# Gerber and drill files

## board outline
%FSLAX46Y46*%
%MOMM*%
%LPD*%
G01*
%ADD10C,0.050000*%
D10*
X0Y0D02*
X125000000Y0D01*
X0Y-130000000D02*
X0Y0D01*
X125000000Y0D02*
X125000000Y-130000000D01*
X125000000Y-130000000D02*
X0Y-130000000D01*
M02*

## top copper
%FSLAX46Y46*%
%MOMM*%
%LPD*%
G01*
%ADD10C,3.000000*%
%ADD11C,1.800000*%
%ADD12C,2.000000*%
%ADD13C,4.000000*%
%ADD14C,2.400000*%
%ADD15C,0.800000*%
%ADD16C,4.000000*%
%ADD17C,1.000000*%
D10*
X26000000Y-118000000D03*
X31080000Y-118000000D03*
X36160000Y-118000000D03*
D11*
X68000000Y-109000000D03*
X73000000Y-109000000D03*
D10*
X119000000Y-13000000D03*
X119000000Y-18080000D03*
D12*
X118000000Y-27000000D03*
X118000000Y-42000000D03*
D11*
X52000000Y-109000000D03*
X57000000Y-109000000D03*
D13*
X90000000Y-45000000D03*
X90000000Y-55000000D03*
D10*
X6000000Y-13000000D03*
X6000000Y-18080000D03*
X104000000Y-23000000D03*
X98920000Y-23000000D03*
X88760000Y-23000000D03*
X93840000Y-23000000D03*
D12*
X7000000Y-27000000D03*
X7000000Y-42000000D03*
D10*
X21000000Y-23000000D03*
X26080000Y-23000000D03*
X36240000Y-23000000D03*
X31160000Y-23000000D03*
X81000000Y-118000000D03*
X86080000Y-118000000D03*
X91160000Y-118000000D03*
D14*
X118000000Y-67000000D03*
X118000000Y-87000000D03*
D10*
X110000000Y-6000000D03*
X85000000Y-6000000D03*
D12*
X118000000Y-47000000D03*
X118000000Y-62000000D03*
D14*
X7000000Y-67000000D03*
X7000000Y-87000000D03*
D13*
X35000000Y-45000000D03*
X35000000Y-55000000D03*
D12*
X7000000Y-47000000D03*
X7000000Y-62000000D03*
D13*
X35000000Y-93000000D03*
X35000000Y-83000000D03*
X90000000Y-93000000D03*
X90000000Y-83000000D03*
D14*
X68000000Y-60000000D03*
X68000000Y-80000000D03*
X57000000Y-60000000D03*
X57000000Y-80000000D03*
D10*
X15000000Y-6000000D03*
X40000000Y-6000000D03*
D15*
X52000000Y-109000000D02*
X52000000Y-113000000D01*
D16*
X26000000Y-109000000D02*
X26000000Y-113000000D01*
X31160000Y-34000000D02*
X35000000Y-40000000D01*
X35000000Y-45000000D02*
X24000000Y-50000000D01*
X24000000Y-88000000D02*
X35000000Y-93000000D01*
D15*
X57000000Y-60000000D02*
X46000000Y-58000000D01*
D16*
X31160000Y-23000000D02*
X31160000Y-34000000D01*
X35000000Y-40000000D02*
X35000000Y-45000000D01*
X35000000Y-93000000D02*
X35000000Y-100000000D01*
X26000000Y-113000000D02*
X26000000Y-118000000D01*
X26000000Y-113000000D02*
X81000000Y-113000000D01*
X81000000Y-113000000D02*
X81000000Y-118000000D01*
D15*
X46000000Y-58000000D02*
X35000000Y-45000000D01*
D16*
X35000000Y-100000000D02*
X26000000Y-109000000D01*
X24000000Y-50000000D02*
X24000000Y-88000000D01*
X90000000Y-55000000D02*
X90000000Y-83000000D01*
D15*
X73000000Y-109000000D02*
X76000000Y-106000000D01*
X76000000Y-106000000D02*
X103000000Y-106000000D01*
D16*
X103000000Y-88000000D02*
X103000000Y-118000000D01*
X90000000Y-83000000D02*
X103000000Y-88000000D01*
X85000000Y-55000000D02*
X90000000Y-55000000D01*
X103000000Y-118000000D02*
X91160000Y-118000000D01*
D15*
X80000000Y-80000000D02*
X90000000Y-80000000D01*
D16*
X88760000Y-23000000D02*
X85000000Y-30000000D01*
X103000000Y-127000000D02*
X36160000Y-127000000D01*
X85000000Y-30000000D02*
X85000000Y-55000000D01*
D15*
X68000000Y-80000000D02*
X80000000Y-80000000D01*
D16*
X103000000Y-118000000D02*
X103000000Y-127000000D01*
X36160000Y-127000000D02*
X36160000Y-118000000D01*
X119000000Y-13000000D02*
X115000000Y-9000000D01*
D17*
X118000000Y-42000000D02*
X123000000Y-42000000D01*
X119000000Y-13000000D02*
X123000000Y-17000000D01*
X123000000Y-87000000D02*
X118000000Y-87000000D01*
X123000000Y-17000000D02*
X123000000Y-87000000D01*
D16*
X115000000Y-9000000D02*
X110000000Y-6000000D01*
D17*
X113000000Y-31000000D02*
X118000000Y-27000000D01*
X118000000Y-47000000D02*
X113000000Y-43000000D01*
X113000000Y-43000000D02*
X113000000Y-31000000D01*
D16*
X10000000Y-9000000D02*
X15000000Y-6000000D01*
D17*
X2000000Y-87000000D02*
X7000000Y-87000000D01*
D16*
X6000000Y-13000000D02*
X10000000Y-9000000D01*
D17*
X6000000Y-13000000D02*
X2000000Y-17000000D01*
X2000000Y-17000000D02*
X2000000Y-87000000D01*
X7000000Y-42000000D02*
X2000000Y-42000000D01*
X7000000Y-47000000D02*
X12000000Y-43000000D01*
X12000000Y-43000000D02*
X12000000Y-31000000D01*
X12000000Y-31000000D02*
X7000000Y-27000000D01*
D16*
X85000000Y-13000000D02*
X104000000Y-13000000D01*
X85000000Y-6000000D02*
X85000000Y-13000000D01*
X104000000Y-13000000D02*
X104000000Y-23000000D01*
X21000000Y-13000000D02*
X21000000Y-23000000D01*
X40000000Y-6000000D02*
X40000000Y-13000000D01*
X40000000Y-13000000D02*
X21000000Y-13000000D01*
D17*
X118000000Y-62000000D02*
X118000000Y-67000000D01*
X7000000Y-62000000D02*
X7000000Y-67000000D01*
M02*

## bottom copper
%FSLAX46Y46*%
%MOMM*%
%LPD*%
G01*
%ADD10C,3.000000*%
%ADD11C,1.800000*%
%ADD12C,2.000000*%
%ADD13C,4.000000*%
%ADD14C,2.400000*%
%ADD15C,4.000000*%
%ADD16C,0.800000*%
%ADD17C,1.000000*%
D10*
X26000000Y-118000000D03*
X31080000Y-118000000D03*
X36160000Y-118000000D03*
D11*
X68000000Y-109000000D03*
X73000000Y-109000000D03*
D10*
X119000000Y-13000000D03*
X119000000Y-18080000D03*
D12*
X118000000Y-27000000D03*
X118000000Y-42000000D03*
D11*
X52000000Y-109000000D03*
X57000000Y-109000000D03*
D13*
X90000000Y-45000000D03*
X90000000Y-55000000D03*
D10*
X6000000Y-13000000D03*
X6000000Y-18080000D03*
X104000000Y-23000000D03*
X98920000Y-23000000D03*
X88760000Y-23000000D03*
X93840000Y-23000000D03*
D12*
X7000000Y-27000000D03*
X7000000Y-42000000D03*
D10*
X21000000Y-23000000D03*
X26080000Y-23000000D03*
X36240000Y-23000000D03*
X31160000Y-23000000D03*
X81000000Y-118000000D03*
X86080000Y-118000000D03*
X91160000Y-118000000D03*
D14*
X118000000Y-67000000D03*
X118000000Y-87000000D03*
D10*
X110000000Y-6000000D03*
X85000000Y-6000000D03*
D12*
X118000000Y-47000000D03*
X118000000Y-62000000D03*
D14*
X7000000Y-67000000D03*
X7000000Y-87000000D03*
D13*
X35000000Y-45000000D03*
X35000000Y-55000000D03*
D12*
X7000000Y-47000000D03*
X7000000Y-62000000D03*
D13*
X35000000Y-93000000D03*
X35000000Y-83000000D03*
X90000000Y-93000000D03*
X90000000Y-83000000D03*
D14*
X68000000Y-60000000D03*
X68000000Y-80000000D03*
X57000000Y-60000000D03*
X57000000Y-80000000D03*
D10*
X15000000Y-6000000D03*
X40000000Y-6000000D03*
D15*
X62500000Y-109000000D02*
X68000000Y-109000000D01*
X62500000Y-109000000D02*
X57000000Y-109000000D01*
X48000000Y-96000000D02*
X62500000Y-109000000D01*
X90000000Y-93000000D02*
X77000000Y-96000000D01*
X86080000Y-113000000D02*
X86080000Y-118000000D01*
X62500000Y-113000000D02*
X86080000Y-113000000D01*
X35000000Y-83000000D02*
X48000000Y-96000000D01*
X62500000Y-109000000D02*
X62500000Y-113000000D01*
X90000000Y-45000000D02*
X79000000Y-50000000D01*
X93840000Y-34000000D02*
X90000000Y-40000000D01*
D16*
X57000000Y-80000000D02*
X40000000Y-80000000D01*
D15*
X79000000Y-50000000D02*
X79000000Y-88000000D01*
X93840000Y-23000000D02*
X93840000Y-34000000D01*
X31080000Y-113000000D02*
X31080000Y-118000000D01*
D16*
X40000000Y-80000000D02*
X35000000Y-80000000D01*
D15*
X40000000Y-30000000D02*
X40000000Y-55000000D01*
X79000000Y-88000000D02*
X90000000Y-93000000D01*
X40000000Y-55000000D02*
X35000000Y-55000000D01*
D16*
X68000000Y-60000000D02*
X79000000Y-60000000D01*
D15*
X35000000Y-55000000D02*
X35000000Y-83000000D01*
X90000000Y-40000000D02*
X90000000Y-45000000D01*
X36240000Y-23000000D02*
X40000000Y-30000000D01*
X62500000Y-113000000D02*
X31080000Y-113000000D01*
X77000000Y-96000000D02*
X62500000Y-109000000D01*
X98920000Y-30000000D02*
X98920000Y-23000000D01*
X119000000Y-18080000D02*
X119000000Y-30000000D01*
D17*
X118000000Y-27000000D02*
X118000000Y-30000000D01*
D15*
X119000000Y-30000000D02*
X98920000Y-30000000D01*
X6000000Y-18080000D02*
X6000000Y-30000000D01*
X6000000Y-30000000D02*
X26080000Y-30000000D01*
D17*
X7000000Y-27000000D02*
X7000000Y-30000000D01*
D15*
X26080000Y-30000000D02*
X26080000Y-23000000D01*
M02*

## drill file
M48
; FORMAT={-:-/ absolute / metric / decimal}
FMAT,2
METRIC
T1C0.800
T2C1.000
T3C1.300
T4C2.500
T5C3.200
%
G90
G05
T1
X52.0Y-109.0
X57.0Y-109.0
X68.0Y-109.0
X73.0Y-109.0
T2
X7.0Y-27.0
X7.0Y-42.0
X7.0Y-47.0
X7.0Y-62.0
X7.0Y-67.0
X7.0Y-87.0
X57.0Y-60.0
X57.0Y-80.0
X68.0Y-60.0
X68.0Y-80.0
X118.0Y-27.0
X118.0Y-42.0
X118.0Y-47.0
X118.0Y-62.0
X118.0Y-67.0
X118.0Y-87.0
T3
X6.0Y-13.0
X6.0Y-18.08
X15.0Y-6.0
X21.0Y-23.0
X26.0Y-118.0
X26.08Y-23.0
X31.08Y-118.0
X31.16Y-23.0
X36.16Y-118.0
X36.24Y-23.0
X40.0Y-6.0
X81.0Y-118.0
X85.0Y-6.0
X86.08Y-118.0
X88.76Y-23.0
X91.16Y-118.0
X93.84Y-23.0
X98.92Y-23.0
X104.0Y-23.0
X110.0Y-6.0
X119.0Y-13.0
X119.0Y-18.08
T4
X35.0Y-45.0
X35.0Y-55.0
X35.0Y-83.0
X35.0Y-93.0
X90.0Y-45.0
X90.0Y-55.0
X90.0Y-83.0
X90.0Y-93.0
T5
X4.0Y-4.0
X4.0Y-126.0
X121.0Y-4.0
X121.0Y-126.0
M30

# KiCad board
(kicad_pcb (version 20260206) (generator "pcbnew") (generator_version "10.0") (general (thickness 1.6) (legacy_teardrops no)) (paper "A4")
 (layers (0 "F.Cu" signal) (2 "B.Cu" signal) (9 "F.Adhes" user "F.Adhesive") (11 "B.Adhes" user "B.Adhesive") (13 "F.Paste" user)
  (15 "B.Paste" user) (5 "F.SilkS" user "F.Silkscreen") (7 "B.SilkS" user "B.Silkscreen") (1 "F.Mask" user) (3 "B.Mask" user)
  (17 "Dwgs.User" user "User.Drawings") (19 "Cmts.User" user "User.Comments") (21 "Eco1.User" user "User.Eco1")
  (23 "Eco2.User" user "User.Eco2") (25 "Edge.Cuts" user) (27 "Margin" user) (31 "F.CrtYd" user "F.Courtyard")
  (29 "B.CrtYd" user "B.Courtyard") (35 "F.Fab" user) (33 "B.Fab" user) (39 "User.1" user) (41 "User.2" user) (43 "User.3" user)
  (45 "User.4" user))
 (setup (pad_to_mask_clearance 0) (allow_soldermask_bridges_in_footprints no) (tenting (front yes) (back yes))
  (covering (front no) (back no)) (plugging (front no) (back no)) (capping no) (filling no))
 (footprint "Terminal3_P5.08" (layer "F.Cu") (at 26 118)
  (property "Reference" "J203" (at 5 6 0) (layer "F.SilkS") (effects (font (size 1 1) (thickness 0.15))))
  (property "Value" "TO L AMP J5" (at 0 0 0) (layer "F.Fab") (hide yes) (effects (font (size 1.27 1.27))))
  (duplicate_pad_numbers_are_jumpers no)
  (pad "1" thru_hole circle (at 0 0) (size 3 3) (drill 1.3) (layers "*.Cu" "*.Mask") (remove_unused_layers no) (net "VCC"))
  (pad "2" thru_hole circle (at 5.08 0) (size 3 3) (drill 1.3) (layers "*.Cu" "*.Mask") (remove_unused_layers no) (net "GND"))
  (pad "3" thru_hole circle (at 10.16 0) (size 3 3) (drill 1.3) (layers "*.Cu" "*.Mask") (remove_unused_layers no) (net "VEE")))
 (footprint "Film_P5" (layer "F.Cu") (at 68 109)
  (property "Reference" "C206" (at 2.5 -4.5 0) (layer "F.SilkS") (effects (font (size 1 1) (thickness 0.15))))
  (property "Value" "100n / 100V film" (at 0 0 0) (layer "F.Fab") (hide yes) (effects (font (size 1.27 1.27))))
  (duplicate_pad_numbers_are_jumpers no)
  (pad "1" thru_hole circle (at 0 0) (size 1.8 1.8) (drill 0.8) (layers "*.Cu" "*.Mask") (remove_unused_layers no) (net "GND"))
  (pad "2" thru_hole circle (at 5 0) (size 1.8 1.8) (drill 0.8) (layers "*.Cu" "*.Mask") (remove_unused_layers no) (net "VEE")))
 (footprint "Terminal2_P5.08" (layer "F.Cu") (at 119 13 -90)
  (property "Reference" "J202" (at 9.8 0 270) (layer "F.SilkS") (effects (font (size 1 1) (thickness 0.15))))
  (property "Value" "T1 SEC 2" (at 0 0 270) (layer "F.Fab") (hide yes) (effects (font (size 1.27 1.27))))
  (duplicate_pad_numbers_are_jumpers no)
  (pad "1" thru_hole circle (at 0 0 270) (size 3 3) (drill 1.3) (layers "*.Cu" "*.Mask") (remove_unused_layers no) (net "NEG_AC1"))
  (pad "2" thru_hole circle (at 5.08 0 270) (size 3 3) (drill 1.3) (layers "*.Cu" "*.Mask") (remove_unused_layers no) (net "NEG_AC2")))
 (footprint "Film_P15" (layer "F.Cu") (at 118 27 -90)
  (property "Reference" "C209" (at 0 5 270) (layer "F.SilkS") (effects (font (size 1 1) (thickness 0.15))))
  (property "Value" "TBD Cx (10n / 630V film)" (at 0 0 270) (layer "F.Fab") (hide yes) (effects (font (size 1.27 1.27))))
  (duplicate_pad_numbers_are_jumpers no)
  (pad "1" thru_hole circle (at 0 0 270) (size 2 2) (drill 1) (layers "*.Cu" "*.Mask") (remove_unused_layers no) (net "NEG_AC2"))
  (pad "2" thru_hole circle (at 15 0 270) (size 2 2) (drill 1) (layers "*.Cu" "*.Mask") (remove_unused_layers no) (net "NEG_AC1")))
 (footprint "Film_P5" (layer "F.Cu") (at 52 109)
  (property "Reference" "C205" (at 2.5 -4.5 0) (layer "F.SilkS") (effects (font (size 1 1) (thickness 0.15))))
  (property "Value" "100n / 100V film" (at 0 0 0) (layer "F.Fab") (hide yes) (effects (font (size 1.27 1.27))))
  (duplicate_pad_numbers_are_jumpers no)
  (pad "1" thru_hole circle (at 0 0) (size 1.8 1.8) (drill 0.8) (layers "*.Cu" "*.Mask") (remove_unused_layers no) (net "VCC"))
  (pad "2" thru_hole circle (at 5 0) (size 1.8 1.8) (drill 0.8) (layers "*.Cu" "*.Mask") (remove_unused_layers no) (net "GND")))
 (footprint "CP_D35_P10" (layer "F.Cu") (at 90 45 -90)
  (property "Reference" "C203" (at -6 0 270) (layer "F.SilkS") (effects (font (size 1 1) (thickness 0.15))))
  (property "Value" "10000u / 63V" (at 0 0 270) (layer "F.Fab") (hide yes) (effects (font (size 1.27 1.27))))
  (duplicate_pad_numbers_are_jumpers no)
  (pad "1" thru_hole circle (at 0 0 270) (size 4 4) (drill 2.5) (layers "*.Cu" "*.Mask") (remove_unused_layers no) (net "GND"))
  (pad "2" thru_hole circle (at 10 0 270) (size 4 4) (drill 2.5) (layers "*.Cu" "*.Mask") (remove_unused_layers no) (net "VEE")))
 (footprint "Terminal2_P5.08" (layer "F.Cu") (at 6 13 -90)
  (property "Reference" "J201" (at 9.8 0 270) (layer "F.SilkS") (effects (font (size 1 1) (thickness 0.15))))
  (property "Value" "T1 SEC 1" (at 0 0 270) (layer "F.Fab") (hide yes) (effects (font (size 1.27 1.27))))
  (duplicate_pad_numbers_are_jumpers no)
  (pad "1" thru_hole circle (at 0 0 270) (size 3 3) (drill 1.3) (layers "*.Cu" "*.Mask") (remove_unused_layers no) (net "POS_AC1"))
  (pad "2" thru_hole circle (at 5.08 0 270) (size 3 3) (drill 1.3) (layers "*.Cu" "*.Mask") (remove_unused_layers no) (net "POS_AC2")))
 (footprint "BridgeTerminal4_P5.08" (layer "F.Cu") (at 104 23 180)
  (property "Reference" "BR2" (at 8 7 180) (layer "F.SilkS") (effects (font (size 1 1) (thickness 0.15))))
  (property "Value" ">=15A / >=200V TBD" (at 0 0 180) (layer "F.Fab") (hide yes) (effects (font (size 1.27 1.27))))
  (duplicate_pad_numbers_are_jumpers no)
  (pad "AC1" thru_hole circle (at 0 0 180) (size 3 3) (drill 1.3) (layers "*.Cu" "*.Mask") (remove_unused_layers no) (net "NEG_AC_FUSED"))
  (pad "AC2" thru_hole circle (at 5.08 0 180) (size 3 3) (drill 1.3) (layers "*.Cu" "*.Mask") (remove_unused_layers no) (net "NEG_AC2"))
  (pad "N" thru_hole circle (at 15.24 0 180) (size 3 3) (drill 1.3) (layers "*.Cu" "*.Mask") (remove_unused_layers no) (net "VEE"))
  (pad "P" thru_hole circle (at 10.16 0 180) (size 3 3) (drill 1.3) (layers "*.Cu" "*.Mask") (remove_unused_layers no) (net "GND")))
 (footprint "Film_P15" (layer "F.Cu") (at 7 27 -90)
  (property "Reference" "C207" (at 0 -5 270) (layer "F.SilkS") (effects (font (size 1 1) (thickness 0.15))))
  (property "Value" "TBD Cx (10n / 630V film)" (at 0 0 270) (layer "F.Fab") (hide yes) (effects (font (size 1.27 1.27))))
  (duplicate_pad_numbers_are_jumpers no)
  (pad "1" thru_hole circle (at 0 0 270) (size 2 2) (drill 1) (layers "*.Cu" "*.Mask") (remove_unused_layers no) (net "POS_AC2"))
  (pad "2" thru_hole circle (at 15 0 270) (size 2 2) (drill 1) (layers "*.Cu" "*.Mask") (remove_unused_layers no) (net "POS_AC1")))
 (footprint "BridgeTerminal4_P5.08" (layer "F.Cu") (at 21 23)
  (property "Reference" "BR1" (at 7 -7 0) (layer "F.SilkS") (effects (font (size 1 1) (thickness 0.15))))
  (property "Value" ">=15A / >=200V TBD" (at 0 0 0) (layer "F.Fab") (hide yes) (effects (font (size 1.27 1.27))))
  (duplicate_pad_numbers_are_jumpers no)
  (pad "AC1" thru_hole circle (at 0 0) (size 3 3) (drill 1.3) (layers "*.Cu" "*.Mask") (remove_unused_layers no) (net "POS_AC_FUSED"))
  (pad "AC2" thru_hole circle (at 5.08 0) (size 3 3) (drill 1.3) (layers "*.Cu" "*.Mask") (remove_unused_layers no) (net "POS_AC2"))
  (pad "N" thru_hole circle (at 15.24 0) (size 3 3) (drill 1.3) (layers "*.Cu" "*.Mask") (remove_unused_layers no) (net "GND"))
  (pad "P" thru_hole circle (at 10.16 0) (size 3 3) (drill 1.3) (layers "*.Cu" "*.Mask") (remove_unused_layers no) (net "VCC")))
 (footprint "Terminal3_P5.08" (layer "F.Cu") (at 81 118)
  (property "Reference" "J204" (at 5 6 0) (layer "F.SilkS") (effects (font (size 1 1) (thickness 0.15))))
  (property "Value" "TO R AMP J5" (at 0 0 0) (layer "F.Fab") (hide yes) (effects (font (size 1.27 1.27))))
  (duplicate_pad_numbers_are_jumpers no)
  (pad "1" thru_hole circle (at 0 0) (size 3 3) (drill 1.3) (layers "*.Cu" "*.Mask") (remove_unused_layers no) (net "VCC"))
  (pad "2" thru_hole circle (at 5.08 0) (size 3 3) (drill 1.3) (layers "*.Cu" "*.Mask") (remove_unused_layers no) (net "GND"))
  (pad "3" thru_hole circle (at 10.16 0) (size 3 3) (drill 1.3) (layers "*.Cu" "*.Mask") (remove_unused_layers no) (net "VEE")))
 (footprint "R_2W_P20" (layer "F.Cu") (at 118 67 -90)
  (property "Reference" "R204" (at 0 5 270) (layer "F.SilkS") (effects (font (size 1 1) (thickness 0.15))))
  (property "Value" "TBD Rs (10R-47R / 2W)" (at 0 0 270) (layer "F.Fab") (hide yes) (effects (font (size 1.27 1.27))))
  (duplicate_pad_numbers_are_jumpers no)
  (pad "1" thru_hole circle (at 0 0 270) (size 2.4 2.4) (drill 1) (layers "*.Cu" "*.Mask") (remove_unused_layers no) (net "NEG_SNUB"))
  (pad "2" thru_hole circle (at 20 0 270) (size 2.4 2.4) (drill 1) (layers "*.Cu" "*.Mask") (remove_unused_layers no) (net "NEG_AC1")))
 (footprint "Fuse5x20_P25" (layer "F.Cu") (at 110 6 180)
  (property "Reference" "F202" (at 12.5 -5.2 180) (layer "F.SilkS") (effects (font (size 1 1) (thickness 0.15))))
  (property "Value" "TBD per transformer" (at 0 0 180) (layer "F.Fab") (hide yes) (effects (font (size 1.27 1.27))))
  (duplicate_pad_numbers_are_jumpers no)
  (pad "1" thru_hole circle (at 0 0 180) (size 3 3) (drill 1.3) (layers "*.Cu" "*.Mask") (remove_unused_layers no) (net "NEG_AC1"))
  (pad "2" thru_hole circle (at 25 0 180) (size 3 3) (drill 1.3) (layers "*.Cu" "*.Mask") (remove_unused_layers no) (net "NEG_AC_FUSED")))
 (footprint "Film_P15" (layer "F.Cu") (at 118 47 -90)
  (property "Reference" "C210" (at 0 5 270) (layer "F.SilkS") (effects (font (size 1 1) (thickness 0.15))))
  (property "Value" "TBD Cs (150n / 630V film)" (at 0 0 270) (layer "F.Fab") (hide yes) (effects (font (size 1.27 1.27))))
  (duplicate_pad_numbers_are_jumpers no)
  (pad "1" thru_hole circle (at 0 0 270) (size 2 2) (drill 1) (layers "*.Cu" "*.Mask") (remove_unused_layers no) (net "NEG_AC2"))
  (pad "2" thru_hole circle (at 15 0 270) (size 2 2) (drill 1) (layers "*.Cu" "*.Mask") (remove_unused_layers no) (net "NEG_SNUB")))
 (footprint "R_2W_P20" (layer "F.Cu") (at 7 67 -90)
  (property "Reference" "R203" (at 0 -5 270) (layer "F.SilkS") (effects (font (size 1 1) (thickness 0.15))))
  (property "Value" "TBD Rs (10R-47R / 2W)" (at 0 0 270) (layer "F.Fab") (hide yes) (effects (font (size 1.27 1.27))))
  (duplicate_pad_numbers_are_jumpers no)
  (pad "1" thru_hole circle (at 0 0 270) (size 2.4 2.4) (drill 1) (layers "*.Cu" "*.Mask") (remove_unused_layers no) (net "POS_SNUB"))
  (pad "2" thru_hole circle (at 20 0 270) (size 2.4 2.4) (drill 1) (layers "*.Cu" "*.Mask") (remove_unused_layers no) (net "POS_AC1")))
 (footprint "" (layer "F.Cu") (at 4 126)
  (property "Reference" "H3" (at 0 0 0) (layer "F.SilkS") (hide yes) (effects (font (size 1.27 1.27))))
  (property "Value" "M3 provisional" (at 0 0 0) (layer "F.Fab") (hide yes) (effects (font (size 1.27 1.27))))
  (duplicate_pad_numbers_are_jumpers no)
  (pad "" np_thru_hole circle (at 0 0) (size 3.2 3.2) (drill 3.2) (layers "*.Cu" "*.Mask")))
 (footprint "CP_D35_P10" (layer "F.Cu") (at 35 45 -90)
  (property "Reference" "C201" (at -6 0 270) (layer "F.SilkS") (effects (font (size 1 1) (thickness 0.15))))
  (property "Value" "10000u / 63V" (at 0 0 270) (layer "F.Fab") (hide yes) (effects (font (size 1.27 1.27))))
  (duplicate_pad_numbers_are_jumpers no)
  (pad "1" thru_hole circle (at 0 0 270) (size 4 4) (drill 2.5) (layers "*.Cu" "*.Mask") (remove_unused_layers no) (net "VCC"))
  (pad "2" thru_hole circle (at 10 0 270) (size 4 4) (drill 2.5) (layers "*.Cu" "*.Mask") (remove_unused_layers no) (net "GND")))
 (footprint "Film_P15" (layer "F.Cu") (at 7 47 -90)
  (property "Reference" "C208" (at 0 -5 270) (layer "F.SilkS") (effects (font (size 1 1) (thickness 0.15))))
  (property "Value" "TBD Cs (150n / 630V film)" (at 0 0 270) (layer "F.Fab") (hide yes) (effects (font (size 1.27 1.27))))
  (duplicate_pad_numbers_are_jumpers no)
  (pad "1" thru_hole circle (at 0 0 270) (size 2 2) (drill 1) (layers "*.Cu" "*.Mask") (remove_unused_layers no) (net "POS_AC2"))
  (pad "2" thru_hole circle (at 15 0 270) (size 2 2) (drill 1) (layers "*.Cu" "*.Mask") (remove_unused_layers no) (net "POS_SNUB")))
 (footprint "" (layer "F.Cu") (at 4 4)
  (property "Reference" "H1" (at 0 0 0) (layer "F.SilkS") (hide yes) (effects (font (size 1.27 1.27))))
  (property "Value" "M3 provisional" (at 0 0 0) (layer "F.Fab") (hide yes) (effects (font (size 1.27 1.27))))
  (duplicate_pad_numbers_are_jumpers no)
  (pad "" np_thru_hole circle (at 0 0) (size 3.2 3.2) (drill 3.2) (layers "*.Cu" "*.Mask")))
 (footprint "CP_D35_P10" (layer "F.Cu") (at 35 93 90)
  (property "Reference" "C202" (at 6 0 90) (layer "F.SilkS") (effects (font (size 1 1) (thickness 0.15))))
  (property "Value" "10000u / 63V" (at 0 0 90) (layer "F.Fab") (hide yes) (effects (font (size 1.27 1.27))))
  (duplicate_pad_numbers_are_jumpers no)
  (pad "1" thru_hole circle (at 0 0 90) (size 4 4) (drill 2.5) (layers "*.Cu" "*.Mask") (remove_unused_layers no) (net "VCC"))
  (pad "2" thru_hole circle (at 10 0 90) (size 4 4) (drill 2.5) (layers "*.Cu" "*.Mask") (remove_unused_layers no) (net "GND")))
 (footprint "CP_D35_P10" (layer "F.Cu") (at 90 93 90)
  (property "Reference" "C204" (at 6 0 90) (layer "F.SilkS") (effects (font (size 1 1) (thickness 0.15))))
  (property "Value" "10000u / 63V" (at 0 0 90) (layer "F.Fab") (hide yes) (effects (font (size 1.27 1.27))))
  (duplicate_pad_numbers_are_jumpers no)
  (pad "1" thru_hole circle (at 0 0 90) (size 4 4) (drill 2.5) (layers "*.Cu" "*.Mask") (remove_unused_layers no) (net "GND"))
  (pad "2" thru_hole circle (at 10 0 90) (size 4 4) (drill 2.5) (layers "*.Cu" "*.Mask") (remove_unused_layers no) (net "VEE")))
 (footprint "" (layer "F.Cu") (at 121 126)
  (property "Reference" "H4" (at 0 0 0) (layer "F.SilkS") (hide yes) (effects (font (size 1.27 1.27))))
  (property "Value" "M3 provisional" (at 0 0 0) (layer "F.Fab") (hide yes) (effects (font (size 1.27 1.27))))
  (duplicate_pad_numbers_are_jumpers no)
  (pad "" np_thru_hole circle (at 0 0) (size 3.2 3.2) (drill 3.2) (layers "*.Cu" "*.Mask")))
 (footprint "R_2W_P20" (layer "F.Cu") (at 68 60 -90)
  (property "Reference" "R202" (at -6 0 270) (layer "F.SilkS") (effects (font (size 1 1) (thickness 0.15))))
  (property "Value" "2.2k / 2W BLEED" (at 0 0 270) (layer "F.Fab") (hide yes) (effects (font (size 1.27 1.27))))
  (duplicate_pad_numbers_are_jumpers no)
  (pad "1" thru_hole circle (at 0 0 270) (size 2.4 2.4) (drill 1) (layers "*.Cu" "*.Mask") (remove_unused_layers no) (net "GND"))
  (pad "2" thru_hole circle (at 20 0 270) (size 2.4 2.4) (drill 1) (layers "*.Cu" "*.Mask") (remove_unused_layers no) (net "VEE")))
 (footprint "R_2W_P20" (layer "F.Cu") (at 57 60 -90)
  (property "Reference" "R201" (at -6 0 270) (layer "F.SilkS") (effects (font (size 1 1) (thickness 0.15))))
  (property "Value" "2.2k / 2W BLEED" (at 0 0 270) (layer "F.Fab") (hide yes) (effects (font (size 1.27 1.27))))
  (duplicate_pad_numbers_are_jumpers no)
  (pad "1" thru_hole circle (at 0 0 270) (size 2.4 2.4) (drill 1) (layers "*.Cu" "*.Mask") (remove_unused_layers no) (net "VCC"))
  (pad "2" thru_hole circle (at 20 0 270) (size 2.4 2.4) (drill 1) (layers "*.Cu" "*.Mask") (remove_unused_layers no) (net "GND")))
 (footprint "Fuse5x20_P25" (layer "F.Cu") (at 15 6)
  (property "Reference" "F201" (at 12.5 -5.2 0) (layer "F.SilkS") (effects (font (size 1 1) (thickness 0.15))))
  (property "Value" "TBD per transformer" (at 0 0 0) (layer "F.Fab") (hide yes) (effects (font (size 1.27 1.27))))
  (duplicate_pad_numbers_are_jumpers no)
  (pad "1" thru_hole circle (at 0 0) (size 3 3) (drill 1.3) (layers "*.Cu" "*.Mask") (remove_unused_layers no) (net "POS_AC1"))
  (pad "2" thru_hole circle (at 25 0) (size 3 3) (drill 1.3) (layers "*.Cu" "*.Mask") (remove_unused_layers no) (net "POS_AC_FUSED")))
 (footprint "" (layer "F.Cu") (at 121 4)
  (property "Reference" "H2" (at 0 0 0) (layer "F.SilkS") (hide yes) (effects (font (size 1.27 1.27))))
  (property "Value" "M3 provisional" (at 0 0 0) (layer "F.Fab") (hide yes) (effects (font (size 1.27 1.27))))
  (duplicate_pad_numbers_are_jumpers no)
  (pad "" np_thru_hole circle (at 0 0) (size 3.2 3.2) (drill 3.2) (layers "*.Cu" "*.Mask")))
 (gr_line (start 0 0) (end 125 0) (stroke (width 0.05) (type default)) (layer "Edge.Cuts"))
 (gr_line (start 0 130) (end 0 0) (stroke (width 0.05) (type default)) (layer "Edge.Cuts"))
 (gr_line (start 125 0) (end 125 130) (stroke (width 0.05) (type default)) (layer "Edge.Cuts"))
 (gr_line (start 125 130) (end 0 130) (stroke (width 0.05) (type default)) (layer "Edge.Cuts"))
 (segment (start 52 109) (end 52 113) (width 0.8) (layer "F.Cu") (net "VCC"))
 (segment (start 26 109) (end 26 113) (width 4) (layer "F.Cu") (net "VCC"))
 (segment (start 31.16 34) (end 35 40) (width 4) (layer "F.Cu") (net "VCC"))
 (segment (start 35 45) (end 24 50) (width 4) (layer "F.Cu") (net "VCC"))
 (segment (start 24 88) (end 35 93) (width 4) (layer "F.Cu") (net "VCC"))
 (segment (start 57 60) (end 46 58) (width 0.8) (layer "F.Cu") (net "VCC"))
 (segment (start 31.16 23) (end 31.16 34) (width 4) (layer "F.Cu") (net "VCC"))
 (segment (start 35 40) (end 35 45) (width 4) (layer "F.Cu") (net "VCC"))
 (segment (start 35 93) (end 35 100) (width 4) (layer "F.Cu") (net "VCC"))
 (segment (start 26 113) (end 26 118) (width 4) (layer "F.Cu") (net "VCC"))
 (segment (start 26 113) (end 81 113) (width 4) (layer "F.Cu") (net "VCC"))
 (segment (start 81 113) (end 81 118) (width 4) (layer "F.Cu") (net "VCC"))
 (segment (start 46 58) (end 35 45) (width 0.8) (layer "F.Cu") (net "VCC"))
 (segment (start 35 100) (end 26 109) (width 4) (layer "F.Cu") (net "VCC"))
 (segment (start 24 50) (end 24 88) (width 4) (layer "F.Cu") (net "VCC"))
 (segment (start 62.5 109) (end 68 109) (width 4) (layer "B.Cu") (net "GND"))
 (segment (start 62.5 109) (end 57 109) (width 4) (layer "B.Cu") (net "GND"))
 (segment (start 48 96) (end 62.5 109) (width 4) (layer "B.Cu") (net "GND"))
 (segment (start 90 93) (end 77 96) (width 4) (layer "B.Cu") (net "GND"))
 (segment (start 86.08 113) (end 86.08 118) (width 4) (layer "B.Cu") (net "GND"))
 (segment (start 62.5 113) (end 86.08 113) (width 4) (layer "B.Cu") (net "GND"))
 (segment (start 35 83) (end 48 96) (width 4) (layer "B.Cu") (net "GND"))
 (segment (start 62.5 109) (end 62.5 113) (width 4) (layer "B.Cu") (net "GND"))
 (segment (start 90 45) (end 79 50) (width 4) (layer "B.Cu") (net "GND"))
 (segment (start 93.84 34) (end 90 40) (width 4) (layer "B.Cu") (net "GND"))
 (segment (start 57 80) (end 40 80) (width 0.8) (layer "B.Cu") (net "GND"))
 (segment (start 79 50) (end 79 88) (width 4) (layer "B.Cu") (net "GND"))
 (segment (start 93.84 23) (end 93.84 34) (width 4) (layer "B.Cu") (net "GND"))
 (segment (start 31.08 113) (end 31.08 118) (width 4) (layer "B.Cu") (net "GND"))
 (segment (start 40 80) (end 35 80) (width 0.8) (layer "B.Cu") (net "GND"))
 (segment (start 40 30) (end 40 55) (width 4) (layer "B.Cu") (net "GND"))
 (segment (start 79 88) (end 90 93) (width 4) (layer "B.Cu") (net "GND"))
 (segment (start 40 55) (end 35 55) (width 4) (layer "B.Cu") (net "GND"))
 (segment (start 68 60) (end 79 60) (width 0.8) (layer "B.Cu") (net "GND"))
 (segment (start 35 55) (end 35 83) (width 4) (layer "B.Cu") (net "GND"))
 (segment (start 90 40) (end 90 45) (width 4) (layer "B.Cu") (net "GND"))
 (segment (start 36.24 23) (end 40 30) (width 4) (layer "B.Cu") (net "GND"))
 (segment (start 62.5 113) (end 31.08 113) (width 4) (layer "B.Cu") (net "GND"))
 (segment (start 77 96) (end 62.5 109) (width 4) (layer "B.Cu") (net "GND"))
 (segment (start 90 55) (end 90 83) (width 4) (layer "F.Cu") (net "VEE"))
 (segment (start 73 109) (end 76 106) (width 0.8) (layer "F.Cu") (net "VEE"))
 (segment (start 76 106) (end 103 106) (width 0.8) (layer "F.Cu") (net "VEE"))
 (segment (start 103 88) (end 103 118) (width 4) (layer "F.Cu") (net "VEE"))
 (segment (start 90 83) (end 103 88) (width 4) (layer "F.Cu") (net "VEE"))
 (segment (start 85 55) (end 90 55) (width 4) (layer "F.Cu") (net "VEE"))
 (segment (start 103 118) (end 91.16 118) (width 4) (layer "F.Cu") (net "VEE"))
 (segment (start 80 80) (end 90 80) (width 0.8) (layer "F.Cu") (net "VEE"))
 (segment (start 88.76 23) (end 85 30) (width 4) (layer "F.Cu") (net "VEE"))
 (segment (start 103 127) (end 36.16 127) (width 4) (layer "F.Cu") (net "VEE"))
 (segment (start 85 30) (end 85 55) (width 4) (layer "F.Cu") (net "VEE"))
 (segment (start 68 80) (end 80 80) (width 0.8) (layer "F.Cu") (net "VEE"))
 (segment (start 103 118) (end 103 127) (width 4) (layer "F.Cu") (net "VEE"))
 (segment (start 36.16 127) (end 36.16 118) (width 4) (layer "F.Cu") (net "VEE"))
 (segment (start 119 13) (end 115 9) (width 4) (layer "F.Cu") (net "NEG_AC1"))
 (segment (start 118 42) (end 123 42) (width 1) (layer "F.Cu") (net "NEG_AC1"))
 (segment (start 119 13) (end 123 17) (width 1) (layer "F.Cu") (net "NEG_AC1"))
 (segment (start 123 87) (end 118 87) (width 1) (layer "F.Cu") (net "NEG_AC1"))
 (segment (start 123 17) (end 123 87) (width 1) (layer "F.Cu") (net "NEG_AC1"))
 (segment (start 115 9) (end 110 6) (width 4) (layer "F.Cu") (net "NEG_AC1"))
 (segment (start 113 31) (end 118 27) (width 1) (layer "F.Cu") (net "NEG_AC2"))
 (segment (start 118 47) (end 113 43) (width 1) (layer "F.Cu") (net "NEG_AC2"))
 (segment (start 113 43) (end 113 31) (width 1) (layer "F.Cu") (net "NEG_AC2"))
 (segment (start 98.92 30) (end 98.92 23) (width 4) (layer "B.Cu") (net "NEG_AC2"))
 (segment (start 119 18.08) (end 119 30) (width 4) (layer "B.Cu") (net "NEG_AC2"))
 (segment (start 118 27) (end 118 30) (width 1) (layer "B.Cu") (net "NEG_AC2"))
 (segment (start 119 30) (end 98.92 30) (width 4) (layer "B.Cu") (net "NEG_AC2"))
 (segment (start 10 9) (end 15 6) (width 4) (layer "F.Cu") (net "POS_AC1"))
 (segment (start 2 87) (end 7 87) (width 1) (layer "F.Cu") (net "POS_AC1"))
 (segment (start 6 13) (end 10 9) (width 4) (layer "F.Cu") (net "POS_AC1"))
 (segment (start 6 13) (end 2 17) (width 1) (layer "F.Cu") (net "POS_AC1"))
 (segment (start 2 17) (end 2 87) (width 1) (layer "F.Cu") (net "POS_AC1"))
 (segment (start 7 42) (end 2 42) (width 1) (layer "F.Cu") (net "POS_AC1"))
 (segment (start 7 47) (end 12 43) (width 1) (layer "F.Cu") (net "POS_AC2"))
 (segment (start 12 43) (end 12 31) (width 1) (layer "F.Cu") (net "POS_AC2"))
 (segment (start 12 31) (end 7 27) (width 1) (layer "F.Cu") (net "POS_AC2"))
 (segment (start 6 18.08) (end 6 30) (width 4) (layer "B.Cu") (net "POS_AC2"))
 (segment (start 6 30) (end 26.08 30) (width 4) (layer "B.Cu") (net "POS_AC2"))
 (segment (start 7 27) (end 7 30) (width 1) (layer "B.Cu") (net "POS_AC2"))
 (segment (start 26.08 30) (end 26.08 23) (width 4) (layer "B.Cu") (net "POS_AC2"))
 (segment (start 85 13) (end 104 13) (width 4) (layer "F.Cu") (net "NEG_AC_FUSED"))
 (segment (start 85 6) (end 85 13) (width 4) (layer "F.Cu") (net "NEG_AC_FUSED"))
 (segment (start 104 13) (end 104 23) (width 4) (layer "F.Cu") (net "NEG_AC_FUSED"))
 (segment (start 21 13) (end 21 23) (width 4) (layer "F.Cu") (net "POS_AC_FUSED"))
 (segment (start 40 6) (end 40 13) (width 4) (layer "F.Cu") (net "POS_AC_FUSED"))
 (segment (start 40 13) (end 21 13) (width 4) (layer "F.Cu") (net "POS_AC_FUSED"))
 (segment (start 118 62) (end 118 67) (width 1) (layer "F.Cu") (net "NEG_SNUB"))
 (segment (start 7 62) (end 7 67) (width 1) (layer "F.Cu") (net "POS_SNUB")))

